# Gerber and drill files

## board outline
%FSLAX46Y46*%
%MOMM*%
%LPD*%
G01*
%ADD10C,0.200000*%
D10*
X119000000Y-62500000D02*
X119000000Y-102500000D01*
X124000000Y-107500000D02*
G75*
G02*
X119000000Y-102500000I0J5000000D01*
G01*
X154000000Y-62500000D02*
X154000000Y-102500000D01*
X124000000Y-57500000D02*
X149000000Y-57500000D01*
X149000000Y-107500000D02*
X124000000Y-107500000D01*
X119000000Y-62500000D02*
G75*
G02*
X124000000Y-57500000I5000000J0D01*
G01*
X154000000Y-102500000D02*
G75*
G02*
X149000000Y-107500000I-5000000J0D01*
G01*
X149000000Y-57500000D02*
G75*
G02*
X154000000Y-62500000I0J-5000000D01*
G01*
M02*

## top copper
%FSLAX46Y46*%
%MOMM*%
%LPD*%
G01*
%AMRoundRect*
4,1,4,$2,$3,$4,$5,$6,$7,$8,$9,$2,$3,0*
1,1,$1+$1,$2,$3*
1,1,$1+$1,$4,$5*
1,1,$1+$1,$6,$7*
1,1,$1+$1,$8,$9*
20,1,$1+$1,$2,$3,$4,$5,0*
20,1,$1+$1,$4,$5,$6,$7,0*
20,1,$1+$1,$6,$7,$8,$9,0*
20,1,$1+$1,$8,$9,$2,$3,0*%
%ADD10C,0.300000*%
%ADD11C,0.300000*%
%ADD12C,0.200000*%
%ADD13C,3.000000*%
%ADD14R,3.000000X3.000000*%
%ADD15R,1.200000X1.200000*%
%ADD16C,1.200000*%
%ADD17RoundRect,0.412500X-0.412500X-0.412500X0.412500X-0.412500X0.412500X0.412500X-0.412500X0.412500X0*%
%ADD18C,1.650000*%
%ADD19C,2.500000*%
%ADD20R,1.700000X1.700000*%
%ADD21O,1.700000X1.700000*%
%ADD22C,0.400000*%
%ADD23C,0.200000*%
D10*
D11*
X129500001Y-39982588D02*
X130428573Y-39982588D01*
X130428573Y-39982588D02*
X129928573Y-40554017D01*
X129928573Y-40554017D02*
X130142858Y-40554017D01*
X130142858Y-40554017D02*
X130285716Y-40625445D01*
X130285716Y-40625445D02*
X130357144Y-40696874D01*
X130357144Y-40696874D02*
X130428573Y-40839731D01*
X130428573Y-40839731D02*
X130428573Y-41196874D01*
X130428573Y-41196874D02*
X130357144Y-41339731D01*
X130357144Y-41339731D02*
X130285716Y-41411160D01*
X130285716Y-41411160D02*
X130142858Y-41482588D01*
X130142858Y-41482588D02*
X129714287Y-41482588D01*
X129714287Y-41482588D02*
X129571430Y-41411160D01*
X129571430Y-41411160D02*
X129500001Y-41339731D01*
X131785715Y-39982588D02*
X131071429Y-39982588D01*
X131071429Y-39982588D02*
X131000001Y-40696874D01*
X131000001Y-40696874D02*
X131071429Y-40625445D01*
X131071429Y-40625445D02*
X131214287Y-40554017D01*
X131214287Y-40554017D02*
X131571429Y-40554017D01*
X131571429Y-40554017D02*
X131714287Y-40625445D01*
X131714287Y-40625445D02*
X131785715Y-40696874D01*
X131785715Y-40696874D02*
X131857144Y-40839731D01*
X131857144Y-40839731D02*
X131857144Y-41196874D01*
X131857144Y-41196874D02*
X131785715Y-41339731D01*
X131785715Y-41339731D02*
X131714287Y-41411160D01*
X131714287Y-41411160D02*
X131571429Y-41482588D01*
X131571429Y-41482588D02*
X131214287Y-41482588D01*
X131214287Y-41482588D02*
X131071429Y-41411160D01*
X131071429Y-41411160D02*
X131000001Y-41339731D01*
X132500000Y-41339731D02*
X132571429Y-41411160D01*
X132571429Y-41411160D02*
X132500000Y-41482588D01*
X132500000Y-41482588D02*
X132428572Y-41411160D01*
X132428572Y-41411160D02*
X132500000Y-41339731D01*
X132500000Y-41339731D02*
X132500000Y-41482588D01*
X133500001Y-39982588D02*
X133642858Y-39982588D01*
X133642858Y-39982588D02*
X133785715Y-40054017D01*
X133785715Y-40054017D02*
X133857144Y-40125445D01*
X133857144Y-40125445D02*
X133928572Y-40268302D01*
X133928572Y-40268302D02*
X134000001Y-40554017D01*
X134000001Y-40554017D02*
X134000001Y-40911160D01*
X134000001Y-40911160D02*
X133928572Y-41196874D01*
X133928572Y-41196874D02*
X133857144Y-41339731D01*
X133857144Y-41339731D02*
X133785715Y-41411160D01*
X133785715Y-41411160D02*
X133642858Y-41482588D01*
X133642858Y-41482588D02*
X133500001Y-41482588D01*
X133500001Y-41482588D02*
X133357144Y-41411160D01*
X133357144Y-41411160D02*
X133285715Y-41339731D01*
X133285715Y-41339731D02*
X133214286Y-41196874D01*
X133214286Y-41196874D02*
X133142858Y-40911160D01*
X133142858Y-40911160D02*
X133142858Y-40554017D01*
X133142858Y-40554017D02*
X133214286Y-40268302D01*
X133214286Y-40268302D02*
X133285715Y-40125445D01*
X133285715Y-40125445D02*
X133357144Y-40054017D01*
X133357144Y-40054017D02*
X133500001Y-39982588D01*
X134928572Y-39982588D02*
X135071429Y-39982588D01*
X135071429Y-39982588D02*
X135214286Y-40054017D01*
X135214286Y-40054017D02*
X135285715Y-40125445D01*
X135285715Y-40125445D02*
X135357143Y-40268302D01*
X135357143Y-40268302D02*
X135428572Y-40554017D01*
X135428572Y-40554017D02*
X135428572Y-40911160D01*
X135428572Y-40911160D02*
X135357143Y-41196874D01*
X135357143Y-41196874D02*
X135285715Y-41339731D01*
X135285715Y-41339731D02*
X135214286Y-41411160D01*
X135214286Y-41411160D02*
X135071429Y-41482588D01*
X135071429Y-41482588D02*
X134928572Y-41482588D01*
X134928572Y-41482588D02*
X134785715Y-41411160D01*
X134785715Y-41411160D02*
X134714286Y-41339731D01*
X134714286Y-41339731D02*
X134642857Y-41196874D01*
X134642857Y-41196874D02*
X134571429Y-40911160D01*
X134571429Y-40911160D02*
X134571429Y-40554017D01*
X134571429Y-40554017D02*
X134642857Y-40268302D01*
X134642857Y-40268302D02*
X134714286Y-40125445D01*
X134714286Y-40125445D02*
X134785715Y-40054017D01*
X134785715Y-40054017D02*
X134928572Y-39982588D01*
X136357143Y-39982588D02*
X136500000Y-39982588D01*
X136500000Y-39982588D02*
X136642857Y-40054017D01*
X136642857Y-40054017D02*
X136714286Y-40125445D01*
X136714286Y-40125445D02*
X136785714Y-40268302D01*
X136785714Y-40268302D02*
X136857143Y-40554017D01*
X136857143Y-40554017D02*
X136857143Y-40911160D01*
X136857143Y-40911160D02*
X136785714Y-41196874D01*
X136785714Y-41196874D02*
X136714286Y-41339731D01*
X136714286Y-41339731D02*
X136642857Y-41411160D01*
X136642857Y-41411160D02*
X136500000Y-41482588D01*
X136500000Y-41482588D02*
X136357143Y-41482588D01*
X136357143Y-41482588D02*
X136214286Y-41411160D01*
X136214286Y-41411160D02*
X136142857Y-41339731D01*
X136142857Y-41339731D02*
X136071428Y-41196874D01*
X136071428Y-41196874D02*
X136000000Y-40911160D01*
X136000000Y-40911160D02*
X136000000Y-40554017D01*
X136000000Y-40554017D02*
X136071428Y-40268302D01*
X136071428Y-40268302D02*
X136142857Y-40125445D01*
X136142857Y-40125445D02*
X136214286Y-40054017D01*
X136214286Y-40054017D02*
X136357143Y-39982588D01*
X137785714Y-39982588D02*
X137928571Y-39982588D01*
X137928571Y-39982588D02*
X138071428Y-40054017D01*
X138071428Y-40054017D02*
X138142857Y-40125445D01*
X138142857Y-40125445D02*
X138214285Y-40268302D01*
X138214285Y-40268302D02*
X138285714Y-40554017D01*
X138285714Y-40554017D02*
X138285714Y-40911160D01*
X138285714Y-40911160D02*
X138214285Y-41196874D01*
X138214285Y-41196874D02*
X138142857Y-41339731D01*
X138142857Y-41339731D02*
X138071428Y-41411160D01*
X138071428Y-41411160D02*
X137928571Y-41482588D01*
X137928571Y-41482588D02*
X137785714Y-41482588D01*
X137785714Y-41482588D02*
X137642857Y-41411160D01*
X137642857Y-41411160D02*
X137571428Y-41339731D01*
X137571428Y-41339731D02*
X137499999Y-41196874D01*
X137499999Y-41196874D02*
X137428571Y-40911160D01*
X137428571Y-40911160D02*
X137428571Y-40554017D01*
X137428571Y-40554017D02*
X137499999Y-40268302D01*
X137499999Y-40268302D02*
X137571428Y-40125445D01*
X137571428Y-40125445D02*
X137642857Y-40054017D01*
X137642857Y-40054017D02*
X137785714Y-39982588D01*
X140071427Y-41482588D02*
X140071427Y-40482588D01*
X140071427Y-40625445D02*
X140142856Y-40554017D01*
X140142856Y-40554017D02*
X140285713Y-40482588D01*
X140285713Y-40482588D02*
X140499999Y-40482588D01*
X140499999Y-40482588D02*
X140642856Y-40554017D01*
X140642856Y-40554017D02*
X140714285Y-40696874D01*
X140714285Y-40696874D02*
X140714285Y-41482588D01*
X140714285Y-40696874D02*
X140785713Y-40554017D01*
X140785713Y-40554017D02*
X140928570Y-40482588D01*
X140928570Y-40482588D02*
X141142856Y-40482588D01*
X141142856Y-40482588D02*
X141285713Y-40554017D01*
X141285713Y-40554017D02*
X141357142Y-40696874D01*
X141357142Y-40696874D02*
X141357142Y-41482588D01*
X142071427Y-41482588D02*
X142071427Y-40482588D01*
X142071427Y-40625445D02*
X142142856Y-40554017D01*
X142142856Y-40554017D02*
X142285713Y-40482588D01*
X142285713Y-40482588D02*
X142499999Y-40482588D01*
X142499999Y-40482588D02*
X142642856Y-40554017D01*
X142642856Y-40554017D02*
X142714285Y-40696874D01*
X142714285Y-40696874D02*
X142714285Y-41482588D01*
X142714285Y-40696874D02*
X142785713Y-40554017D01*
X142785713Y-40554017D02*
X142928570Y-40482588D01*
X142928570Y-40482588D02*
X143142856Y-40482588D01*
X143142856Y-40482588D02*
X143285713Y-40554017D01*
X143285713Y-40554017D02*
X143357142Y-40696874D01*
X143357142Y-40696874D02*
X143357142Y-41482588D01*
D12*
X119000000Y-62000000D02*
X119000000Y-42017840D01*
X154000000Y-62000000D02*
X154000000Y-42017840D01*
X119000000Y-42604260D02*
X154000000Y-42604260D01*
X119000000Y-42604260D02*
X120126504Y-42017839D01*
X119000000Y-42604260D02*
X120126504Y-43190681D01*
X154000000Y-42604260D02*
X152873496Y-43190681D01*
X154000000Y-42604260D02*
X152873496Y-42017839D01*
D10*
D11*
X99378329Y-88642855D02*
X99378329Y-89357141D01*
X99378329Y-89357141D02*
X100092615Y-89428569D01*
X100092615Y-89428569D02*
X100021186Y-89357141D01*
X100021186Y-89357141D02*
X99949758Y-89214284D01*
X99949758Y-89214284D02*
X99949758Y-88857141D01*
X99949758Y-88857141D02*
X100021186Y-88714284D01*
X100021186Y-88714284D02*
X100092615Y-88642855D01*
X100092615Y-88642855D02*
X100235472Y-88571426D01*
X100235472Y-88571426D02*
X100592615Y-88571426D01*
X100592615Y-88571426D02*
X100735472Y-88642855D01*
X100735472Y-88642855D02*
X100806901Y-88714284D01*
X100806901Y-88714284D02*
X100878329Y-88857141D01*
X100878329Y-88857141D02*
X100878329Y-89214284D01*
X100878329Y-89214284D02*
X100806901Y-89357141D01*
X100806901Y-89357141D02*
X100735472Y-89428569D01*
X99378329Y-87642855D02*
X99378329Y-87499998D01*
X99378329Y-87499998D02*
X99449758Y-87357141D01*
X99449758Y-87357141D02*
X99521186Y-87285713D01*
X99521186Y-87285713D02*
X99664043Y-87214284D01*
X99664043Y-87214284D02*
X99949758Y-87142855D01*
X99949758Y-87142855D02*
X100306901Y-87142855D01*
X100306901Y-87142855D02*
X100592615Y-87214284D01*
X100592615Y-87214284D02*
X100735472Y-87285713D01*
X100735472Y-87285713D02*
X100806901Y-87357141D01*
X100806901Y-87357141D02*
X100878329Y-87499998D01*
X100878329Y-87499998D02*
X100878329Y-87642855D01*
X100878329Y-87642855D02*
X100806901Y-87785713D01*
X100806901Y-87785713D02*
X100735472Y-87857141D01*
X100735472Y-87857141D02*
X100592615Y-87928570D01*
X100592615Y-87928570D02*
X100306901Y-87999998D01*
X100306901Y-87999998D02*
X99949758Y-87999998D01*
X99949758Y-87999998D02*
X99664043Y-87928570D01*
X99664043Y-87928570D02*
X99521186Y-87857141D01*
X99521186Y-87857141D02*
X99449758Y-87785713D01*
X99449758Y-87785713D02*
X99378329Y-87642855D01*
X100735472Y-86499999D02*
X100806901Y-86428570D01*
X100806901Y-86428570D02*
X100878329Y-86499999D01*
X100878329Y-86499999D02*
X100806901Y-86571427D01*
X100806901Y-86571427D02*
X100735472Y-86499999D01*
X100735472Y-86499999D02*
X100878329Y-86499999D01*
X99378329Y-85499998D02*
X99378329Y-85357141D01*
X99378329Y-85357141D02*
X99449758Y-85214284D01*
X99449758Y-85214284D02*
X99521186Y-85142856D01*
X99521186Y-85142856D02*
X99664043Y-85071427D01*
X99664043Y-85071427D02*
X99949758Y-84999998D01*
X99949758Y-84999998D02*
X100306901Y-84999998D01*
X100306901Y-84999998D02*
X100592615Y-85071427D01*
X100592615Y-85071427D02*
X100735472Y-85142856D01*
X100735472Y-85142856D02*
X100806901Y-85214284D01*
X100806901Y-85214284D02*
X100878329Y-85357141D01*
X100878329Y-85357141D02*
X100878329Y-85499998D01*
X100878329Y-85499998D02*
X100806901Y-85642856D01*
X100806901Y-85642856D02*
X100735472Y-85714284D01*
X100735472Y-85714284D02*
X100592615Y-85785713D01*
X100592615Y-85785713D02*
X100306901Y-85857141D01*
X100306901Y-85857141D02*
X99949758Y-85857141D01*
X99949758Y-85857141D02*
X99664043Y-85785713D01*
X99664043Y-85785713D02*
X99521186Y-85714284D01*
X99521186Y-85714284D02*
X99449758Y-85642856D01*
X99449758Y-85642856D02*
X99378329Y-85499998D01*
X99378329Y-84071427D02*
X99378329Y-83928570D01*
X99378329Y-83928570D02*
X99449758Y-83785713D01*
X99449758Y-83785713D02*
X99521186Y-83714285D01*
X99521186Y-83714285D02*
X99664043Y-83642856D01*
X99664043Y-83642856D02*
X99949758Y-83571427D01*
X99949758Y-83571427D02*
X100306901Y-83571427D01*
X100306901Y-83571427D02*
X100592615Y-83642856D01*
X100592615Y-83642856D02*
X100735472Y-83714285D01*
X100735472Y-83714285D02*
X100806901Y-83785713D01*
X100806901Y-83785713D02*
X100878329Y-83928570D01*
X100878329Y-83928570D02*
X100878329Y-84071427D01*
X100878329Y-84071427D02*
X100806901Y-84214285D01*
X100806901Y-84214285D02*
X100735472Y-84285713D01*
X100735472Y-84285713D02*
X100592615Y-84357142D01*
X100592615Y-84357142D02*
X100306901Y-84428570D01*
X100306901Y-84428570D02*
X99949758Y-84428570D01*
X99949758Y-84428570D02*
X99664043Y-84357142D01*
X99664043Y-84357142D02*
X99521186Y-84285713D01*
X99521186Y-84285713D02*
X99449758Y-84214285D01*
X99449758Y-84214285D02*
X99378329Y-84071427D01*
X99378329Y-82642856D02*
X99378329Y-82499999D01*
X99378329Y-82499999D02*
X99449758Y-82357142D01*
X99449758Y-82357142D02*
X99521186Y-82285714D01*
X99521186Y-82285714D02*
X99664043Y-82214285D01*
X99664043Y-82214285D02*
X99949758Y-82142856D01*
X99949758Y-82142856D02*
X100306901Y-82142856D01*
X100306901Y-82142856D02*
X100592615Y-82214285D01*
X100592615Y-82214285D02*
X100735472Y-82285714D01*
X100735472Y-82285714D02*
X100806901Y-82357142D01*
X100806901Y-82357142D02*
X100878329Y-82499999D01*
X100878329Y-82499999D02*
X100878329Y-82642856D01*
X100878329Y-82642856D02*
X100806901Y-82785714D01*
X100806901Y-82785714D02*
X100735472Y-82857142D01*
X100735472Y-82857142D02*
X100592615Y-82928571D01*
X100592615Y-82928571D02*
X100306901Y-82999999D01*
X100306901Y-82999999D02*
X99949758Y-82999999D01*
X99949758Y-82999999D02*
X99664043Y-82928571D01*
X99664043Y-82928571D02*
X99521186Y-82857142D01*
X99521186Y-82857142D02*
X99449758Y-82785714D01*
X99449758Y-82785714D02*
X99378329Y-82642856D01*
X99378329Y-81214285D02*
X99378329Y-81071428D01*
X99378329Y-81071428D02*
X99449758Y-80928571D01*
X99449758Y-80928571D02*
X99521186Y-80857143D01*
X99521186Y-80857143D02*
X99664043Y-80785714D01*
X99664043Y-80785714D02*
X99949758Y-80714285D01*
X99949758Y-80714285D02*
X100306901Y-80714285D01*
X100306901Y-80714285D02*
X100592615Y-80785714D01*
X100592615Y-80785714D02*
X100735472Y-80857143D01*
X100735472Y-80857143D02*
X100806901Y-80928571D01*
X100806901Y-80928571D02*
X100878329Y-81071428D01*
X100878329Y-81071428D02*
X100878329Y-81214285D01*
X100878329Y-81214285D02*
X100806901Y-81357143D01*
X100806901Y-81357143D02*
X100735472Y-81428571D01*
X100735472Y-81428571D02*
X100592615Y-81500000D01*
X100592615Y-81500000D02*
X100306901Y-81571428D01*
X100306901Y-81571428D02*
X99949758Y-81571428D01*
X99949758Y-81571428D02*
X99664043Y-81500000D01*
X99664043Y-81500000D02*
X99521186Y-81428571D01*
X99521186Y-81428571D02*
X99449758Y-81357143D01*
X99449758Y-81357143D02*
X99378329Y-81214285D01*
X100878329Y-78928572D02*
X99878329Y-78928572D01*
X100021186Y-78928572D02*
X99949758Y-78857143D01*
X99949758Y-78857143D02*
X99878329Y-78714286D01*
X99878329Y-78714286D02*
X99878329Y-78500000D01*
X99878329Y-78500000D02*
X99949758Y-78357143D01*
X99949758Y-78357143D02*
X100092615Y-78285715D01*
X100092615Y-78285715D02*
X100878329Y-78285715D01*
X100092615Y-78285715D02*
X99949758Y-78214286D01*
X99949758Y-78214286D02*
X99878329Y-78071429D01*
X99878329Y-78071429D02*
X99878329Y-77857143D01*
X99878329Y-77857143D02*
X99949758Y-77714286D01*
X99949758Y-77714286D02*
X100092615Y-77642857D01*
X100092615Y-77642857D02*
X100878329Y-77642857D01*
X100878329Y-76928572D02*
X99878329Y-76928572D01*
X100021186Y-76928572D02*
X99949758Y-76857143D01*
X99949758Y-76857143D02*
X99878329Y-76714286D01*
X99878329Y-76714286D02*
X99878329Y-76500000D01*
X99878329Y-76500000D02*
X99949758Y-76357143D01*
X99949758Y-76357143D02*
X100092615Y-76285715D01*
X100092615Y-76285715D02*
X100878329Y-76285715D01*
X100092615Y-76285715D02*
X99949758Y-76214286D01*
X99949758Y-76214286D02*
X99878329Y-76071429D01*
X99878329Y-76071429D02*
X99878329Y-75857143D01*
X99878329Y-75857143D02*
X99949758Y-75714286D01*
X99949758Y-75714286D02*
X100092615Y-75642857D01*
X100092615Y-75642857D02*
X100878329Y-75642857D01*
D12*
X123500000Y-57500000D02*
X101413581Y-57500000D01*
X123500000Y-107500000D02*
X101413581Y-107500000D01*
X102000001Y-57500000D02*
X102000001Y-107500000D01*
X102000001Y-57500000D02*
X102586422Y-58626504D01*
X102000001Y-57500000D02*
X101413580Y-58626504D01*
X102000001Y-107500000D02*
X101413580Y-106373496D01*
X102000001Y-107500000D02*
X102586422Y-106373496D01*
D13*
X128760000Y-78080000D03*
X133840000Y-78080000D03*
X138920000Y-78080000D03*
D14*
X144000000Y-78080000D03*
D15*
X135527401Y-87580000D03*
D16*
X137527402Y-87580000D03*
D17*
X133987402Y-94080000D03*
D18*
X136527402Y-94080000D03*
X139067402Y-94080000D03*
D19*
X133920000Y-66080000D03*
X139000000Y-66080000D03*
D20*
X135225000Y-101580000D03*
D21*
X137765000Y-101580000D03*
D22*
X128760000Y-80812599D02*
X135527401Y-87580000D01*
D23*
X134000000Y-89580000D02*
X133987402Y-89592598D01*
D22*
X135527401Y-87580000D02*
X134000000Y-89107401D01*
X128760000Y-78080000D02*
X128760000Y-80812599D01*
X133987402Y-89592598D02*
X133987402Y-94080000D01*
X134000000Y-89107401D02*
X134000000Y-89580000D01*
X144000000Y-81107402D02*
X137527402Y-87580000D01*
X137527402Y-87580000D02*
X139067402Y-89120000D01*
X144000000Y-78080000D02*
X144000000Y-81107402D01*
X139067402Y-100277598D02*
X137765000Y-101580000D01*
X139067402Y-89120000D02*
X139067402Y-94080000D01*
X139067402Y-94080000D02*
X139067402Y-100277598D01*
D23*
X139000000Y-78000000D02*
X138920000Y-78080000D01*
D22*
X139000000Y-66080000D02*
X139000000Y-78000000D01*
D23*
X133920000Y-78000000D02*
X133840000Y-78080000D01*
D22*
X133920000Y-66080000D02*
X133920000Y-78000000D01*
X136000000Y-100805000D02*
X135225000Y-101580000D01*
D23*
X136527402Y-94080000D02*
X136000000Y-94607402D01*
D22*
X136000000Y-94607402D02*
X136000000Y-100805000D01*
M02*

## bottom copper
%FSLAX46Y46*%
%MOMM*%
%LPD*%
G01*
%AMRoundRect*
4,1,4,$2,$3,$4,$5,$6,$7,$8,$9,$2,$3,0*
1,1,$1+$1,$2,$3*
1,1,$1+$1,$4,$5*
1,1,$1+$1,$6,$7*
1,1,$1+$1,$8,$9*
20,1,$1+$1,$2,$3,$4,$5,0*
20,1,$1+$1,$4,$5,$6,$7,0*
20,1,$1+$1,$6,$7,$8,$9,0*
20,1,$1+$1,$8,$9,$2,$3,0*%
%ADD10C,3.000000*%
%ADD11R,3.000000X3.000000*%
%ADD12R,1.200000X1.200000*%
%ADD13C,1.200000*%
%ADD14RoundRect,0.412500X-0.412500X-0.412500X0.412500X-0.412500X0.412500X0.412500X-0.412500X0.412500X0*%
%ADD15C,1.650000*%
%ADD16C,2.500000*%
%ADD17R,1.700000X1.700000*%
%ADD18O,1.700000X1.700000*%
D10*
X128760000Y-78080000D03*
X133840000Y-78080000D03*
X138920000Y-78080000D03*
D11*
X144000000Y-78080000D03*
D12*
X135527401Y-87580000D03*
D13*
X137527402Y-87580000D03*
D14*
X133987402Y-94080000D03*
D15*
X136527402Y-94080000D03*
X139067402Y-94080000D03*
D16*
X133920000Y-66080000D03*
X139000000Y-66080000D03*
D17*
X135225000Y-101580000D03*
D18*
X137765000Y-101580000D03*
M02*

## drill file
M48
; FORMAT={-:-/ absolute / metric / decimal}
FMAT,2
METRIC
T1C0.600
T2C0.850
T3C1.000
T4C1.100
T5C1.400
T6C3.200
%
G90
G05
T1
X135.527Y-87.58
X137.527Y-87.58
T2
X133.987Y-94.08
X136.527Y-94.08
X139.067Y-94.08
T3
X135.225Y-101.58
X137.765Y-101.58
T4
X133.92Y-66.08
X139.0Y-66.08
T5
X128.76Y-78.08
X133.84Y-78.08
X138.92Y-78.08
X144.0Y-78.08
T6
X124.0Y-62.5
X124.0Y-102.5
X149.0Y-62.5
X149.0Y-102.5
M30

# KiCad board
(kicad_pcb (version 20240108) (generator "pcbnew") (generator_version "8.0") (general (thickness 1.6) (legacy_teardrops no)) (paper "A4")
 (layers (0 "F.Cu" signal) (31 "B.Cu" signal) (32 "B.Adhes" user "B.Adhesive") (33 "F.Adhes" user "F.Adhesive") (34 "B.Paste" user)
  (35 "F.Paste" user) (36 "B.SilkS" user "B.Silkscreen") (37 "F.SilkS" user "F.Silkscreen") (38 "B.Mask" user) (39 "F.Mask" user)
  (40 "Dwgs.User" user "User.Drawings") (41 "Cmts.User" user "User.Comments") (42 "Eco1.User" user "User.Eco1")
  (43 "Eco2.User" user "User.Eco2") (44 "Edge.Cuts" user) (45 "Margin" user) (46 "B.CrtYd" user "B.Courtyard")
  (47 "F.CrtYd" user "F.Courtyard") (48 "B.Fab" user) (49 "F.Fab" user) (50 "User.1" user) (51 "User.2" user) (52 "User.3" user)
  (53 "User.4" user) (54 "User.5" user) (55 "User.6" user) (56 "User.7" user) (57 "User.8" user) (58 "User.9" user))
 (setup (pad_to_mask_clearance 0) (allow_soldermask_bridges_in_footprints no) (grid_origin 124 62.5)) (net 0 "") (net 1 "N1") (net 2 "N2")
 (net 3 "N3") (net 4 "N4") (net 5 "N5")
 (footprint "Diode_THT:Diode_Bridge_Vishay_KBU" (layer "F.Cu") (at 128.76 78.08)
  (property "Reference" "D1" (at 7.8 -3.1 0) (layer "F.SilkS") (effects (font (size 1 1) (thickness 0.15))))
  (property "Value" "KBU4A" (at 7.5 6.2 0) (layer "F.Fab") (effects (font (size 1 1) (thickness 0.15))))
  (pad "1" thru_hole circle (at 0 0) (size 3 3) (drill 1.4) (layers "*.Cu" "*.Mask") (remove_unused_layers no) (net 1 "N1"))
  (pad "2" thru_hole circle (at 5.08 0) (size 3 3) (drill 1.4) (layers "*.Cu" "*.Mask") (remove_unused_layers no) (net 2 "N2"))
  (pad "3" thru_hole circle (at 10.16 0) (size 3 3) (drill 1.4) (layers "*.Cu" "*.Mask") (remove_unused_layers no) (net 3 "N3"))
  (pad "4" thru_hole rect (at 15.24 0) (size 3 3) (drill 1.4) (layers "*.Cu" "*.Mask") (remove_unused_layers no) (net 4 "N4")))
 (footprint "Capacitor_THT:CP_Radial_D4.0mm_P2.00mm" (layer "F.Cu") (at 135.527401 87.58)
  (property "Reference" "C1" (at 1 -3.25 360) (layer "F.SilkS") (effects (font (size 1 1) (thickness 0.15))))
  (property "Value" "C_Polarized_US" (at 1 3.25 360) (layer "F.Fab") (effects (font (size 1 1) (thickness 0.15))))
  (pad "1" thru_hole rect (at 0 0) (size 1.2 1.2) (drill 0.6) (layers "*.Cu" "*.Mask") (remove_unused_layers no) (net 1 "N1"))
  (pad "2" thru_hole circle (at 2.000001 0) (size 1.2 1.2) (drill 0.6) (layers "*.Cu" "*.Mask") (remove_unused_layers no) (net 4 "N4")))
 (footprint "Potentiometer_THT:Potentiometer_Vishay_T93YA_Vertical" (layer "F.Cu") (at 133.987402 94.08)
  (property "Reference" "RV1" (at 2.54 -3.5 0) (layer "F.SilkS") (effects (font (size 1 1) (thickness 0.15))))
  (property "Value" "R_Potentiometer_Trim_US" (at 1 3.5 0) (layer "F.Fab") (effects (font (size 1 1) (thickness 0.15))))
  (pad "1" thru_hole roundrect (at 0 0) (size 1.65 1.65) (drill 0.85) (layers "*.Cu" "*.Mask") (remove_unused_layers no)
   (roundrect_rratio 0.25) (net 1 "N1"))
  (pad "2" thru_hole circle (at 2.54 0) (size 1.65 1.65) (drill 0.85) (layers "*.Cu" "*.Mask") (remove_unused_layers no) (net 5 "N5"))
  (pad "3" thru_hole circle (at 5.08 0) (size 1.65 1.65) (drill 0.85) (layers "*.Cu" "*.Mask") (remove_unused_layers no) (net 4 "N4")))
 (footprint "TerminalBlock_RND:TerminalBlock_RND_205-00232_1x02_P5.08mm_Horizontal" (layer "F.Cu") (at 133.92 66.08)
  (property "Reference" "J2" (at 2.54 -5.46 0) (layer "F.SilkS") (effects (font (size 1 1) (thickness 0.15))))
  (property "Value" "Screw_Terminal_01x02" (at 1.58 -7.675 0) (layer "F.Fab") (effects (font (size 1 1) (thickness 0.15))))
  (pad "1" thru_hole circle (at 0 0) (size 2.5 2.5) (drill 1.1) (layers "*.Cu" "*.Mask") (remove_unused_layers no) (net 2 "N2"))
  (pad "2" thru_hole circle (at 5.08 0) (size 2.5 2.5) (drill 1.1) (layers "*.Cu" "*.Mask") (remove_unused_layers no) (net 3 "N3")))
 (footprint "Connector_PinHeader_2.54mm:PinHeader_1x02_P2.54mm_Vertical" (layer "F.Cu") (at 135.225 101.58 90)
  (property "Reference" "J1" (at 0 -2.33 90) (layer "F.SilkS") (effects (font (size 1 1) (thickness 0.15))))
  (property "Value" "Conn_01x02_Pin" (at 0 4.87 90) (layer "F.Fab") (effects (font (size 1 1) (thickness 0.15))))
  (pad "1" thru_hole rect (at 0 0 90) (size 1.7 1.7) (drill 1) (layers "*.Cu" "*.Mask") (remove_unused_layers no) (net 5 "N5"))
  (pad "2" thru_hole oval (at 0 2.54 90) (size 1.7 1.7) (drill 1) (layers "*.Cu" "*.Mask") (remove_unused_layers no) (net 4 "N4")))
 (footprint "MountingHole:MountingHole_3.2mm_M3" (layer "F.Cu") (at 124 102.5)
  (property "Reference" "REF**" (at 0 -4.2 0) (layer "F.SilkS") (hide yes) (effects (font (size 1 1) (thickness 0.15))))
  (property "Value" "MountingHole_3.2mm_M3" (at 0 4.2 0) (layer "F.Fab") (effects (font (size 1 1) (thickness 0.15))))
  (pad "" np_thru_hole circle (at 0 0) (size 3.2 3.2) (drill 3.2) (layers "F&B.Cu" "*.Mask")))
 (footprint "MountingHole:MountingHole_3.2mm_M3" (layer "F.Cu") (at 149 62.5)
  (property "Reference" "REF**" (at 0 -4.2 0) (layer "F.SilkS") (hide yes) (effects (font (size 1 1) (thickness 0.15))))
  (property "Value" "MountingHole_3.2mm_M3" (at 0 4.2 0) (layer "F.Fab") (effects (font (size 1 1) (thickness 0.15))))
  (pad "" np_thru_hole circle (at 0 0) (size 3.2 3.2) (drill 3.2) (layers "*.Cu" "*.Mask")))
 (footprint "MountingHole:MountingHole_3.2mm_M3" (layer "F.Cu") (at 124 62.5)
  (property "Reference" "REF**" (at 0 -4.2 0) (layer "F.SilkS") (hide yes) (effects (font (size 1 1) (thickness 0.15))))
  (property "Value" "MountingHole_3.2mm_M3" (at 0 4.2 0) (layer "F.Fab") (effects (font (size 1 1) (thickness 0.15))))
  (pad "" np_thru_hole circle (at 0 0) (size 3.2 3.2) (drill 3.2) (layers "F&B.Cu" "*.Mask")))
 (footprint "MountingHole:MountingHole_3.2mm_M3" (layer "F.Cu") (at 149 102.5)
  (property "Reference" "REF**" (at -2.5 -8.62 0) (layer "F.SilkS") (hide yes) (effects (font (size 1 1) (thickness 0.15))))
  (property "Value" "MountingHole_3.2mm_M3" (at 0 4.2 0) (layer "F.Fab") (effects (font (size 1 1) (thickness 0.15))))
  (pad "" np_thru_hole circle (at 0 0) (size 3.2 3.2) (drill 3.2) (layers "F&B.Cu" "*.Mask")))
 (gr_line (start 119 62.5) (end 119 102.5) (stroke (width 0.2) (type default)) (layer "Edge.Cuts"))
 (gr_arc (start 124 107.5) (mid 120.464466 106.035534) (end 119 102.5) (stroke (width 0.2) (type default)) (layer "Edge.Cuts"))
 (gr_line (start 154 62.5) (end 154 102.5) (stroke (width 0.2) (type default)) (layer "Edge.Cuts"))
 (gr_line (start 124 57.5) (end 149 57.5) (stroke (width 0.2) (type default)) (layer "Edge.Cuts"))
 (gr_line (start 149 107.5) (end 124 107.5) (stroke (width 0.2) (type default)) (layer "Edge.Cuts"))
 (gr_arc (start 119 62.5) (mid 120.464466 58.964466) (end 124 57.5) (stroke (width 0.2) (type default)) (layer "Edge.Cuts"))
 (gr_arc (start 154 102.5) (mid 152.535534 106.035534) (end 149 107.5) (stroke (width 0.2) (type default)) (layer "Edge.Cuts"))
 (gr_arc (start 149 57.5) (mid 152.535534 58.964466) (end 154 62.5) (stroke (width 0.2) (type default)) (layer "Edge.Cuts"))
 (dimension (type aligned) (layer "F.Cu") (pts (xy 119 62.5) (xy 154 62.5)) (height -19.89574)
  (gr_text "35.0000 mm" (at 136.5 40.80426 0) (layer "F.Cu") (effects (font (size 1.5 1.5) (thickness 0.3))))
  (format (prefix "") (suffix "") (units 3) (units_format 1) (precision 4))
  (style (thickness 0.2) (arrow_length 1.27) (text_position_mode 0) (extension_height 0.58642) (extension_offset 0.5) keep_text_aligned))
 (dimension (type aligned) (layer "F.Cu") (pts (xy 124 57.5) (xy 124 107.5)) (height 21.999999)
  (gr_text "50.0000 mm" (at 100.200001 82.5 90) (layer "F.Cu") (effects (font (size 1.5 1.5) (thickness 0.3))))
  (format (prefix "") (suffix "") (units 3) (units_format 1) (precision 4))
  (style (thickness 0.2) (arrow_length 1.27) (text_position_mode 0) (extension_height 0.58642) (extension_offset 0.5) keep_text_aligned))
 (segment (start 128.76 80.812599) (end 135.527401 87.58) (width 0.4) (layer "F.Cu") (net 1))
 (segment (start 134 89.58) (end 133.987402 89.592598) (width 0.2) (layer "F.Cu") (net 1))
 (segment (start 135.527401 87.58) (end 134 89.107401) (width 0.4) (layer "F.Cu") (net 1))
 (segment (start 128.76 78.08) (end 128.76 80.812599) (width 0.4) (layer "F.Cu") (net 1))
 (segment (start 133.987402 89.592598) (end 133.987402 94.08) (width 0.4) (layer "F.Cu") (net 1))
 (segment (start 134 89.107401) (end 134 89.58) (width 0.4) (layer "F.Cu") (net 1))
 (segment (start 144 81.107402) (end 137.527402 87.58) (width 0.4) (layer "F.Cu") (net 4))
 (segment (start 137.527402 87.58) (end 139.067402 89.12) (width 0.4) (layer "F.Cu") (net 4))
 (segment (start 144 78.08) (end 144 81.107402) (width 0.4) (layer "F.Cu") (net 4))
 (segment (start 139.067402 100.277598) (end 137.765 101.58) (width 0.4) (layer "F.Cu") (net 4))
 (segment (start 139.067402 89.12) (end 139.067402 94.08) (width 0.4) (layer "F.Cu") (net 4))
 (segment (start 139.067402 94.08) (end 139.067402 100.277598) (width 0.4) (layer "F.Cu") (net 4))
 (segment (start 139 78) (end 138.92 78.08) (width 0.2) (layer "F.Cu") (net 3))
 (segment (start 139 66.08) (end 139 78) (width 0.4) (layer "F.Cu") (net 3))
 (segment (start 133.92 78) (end 133.84 78.08) (width 0.2) (layer "F.Cu") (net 2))
 (segment (start 133.92 66.08) (end 133.92 78) (width 0.4) (layer "F.Cu") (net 2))
 (segment (start 136 100.805) (end 135.225 101.58) (width 0.4) (layer "F.Cu") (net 5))
 (segment (start 136.527402 94.08) (end 136 94.607402) (width 0.2) (layer "F.Cu") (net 5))
 (segment (start 136 94.607402) (end 136 100.805) (width 0.4) (layer "F.Cu") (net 5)))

